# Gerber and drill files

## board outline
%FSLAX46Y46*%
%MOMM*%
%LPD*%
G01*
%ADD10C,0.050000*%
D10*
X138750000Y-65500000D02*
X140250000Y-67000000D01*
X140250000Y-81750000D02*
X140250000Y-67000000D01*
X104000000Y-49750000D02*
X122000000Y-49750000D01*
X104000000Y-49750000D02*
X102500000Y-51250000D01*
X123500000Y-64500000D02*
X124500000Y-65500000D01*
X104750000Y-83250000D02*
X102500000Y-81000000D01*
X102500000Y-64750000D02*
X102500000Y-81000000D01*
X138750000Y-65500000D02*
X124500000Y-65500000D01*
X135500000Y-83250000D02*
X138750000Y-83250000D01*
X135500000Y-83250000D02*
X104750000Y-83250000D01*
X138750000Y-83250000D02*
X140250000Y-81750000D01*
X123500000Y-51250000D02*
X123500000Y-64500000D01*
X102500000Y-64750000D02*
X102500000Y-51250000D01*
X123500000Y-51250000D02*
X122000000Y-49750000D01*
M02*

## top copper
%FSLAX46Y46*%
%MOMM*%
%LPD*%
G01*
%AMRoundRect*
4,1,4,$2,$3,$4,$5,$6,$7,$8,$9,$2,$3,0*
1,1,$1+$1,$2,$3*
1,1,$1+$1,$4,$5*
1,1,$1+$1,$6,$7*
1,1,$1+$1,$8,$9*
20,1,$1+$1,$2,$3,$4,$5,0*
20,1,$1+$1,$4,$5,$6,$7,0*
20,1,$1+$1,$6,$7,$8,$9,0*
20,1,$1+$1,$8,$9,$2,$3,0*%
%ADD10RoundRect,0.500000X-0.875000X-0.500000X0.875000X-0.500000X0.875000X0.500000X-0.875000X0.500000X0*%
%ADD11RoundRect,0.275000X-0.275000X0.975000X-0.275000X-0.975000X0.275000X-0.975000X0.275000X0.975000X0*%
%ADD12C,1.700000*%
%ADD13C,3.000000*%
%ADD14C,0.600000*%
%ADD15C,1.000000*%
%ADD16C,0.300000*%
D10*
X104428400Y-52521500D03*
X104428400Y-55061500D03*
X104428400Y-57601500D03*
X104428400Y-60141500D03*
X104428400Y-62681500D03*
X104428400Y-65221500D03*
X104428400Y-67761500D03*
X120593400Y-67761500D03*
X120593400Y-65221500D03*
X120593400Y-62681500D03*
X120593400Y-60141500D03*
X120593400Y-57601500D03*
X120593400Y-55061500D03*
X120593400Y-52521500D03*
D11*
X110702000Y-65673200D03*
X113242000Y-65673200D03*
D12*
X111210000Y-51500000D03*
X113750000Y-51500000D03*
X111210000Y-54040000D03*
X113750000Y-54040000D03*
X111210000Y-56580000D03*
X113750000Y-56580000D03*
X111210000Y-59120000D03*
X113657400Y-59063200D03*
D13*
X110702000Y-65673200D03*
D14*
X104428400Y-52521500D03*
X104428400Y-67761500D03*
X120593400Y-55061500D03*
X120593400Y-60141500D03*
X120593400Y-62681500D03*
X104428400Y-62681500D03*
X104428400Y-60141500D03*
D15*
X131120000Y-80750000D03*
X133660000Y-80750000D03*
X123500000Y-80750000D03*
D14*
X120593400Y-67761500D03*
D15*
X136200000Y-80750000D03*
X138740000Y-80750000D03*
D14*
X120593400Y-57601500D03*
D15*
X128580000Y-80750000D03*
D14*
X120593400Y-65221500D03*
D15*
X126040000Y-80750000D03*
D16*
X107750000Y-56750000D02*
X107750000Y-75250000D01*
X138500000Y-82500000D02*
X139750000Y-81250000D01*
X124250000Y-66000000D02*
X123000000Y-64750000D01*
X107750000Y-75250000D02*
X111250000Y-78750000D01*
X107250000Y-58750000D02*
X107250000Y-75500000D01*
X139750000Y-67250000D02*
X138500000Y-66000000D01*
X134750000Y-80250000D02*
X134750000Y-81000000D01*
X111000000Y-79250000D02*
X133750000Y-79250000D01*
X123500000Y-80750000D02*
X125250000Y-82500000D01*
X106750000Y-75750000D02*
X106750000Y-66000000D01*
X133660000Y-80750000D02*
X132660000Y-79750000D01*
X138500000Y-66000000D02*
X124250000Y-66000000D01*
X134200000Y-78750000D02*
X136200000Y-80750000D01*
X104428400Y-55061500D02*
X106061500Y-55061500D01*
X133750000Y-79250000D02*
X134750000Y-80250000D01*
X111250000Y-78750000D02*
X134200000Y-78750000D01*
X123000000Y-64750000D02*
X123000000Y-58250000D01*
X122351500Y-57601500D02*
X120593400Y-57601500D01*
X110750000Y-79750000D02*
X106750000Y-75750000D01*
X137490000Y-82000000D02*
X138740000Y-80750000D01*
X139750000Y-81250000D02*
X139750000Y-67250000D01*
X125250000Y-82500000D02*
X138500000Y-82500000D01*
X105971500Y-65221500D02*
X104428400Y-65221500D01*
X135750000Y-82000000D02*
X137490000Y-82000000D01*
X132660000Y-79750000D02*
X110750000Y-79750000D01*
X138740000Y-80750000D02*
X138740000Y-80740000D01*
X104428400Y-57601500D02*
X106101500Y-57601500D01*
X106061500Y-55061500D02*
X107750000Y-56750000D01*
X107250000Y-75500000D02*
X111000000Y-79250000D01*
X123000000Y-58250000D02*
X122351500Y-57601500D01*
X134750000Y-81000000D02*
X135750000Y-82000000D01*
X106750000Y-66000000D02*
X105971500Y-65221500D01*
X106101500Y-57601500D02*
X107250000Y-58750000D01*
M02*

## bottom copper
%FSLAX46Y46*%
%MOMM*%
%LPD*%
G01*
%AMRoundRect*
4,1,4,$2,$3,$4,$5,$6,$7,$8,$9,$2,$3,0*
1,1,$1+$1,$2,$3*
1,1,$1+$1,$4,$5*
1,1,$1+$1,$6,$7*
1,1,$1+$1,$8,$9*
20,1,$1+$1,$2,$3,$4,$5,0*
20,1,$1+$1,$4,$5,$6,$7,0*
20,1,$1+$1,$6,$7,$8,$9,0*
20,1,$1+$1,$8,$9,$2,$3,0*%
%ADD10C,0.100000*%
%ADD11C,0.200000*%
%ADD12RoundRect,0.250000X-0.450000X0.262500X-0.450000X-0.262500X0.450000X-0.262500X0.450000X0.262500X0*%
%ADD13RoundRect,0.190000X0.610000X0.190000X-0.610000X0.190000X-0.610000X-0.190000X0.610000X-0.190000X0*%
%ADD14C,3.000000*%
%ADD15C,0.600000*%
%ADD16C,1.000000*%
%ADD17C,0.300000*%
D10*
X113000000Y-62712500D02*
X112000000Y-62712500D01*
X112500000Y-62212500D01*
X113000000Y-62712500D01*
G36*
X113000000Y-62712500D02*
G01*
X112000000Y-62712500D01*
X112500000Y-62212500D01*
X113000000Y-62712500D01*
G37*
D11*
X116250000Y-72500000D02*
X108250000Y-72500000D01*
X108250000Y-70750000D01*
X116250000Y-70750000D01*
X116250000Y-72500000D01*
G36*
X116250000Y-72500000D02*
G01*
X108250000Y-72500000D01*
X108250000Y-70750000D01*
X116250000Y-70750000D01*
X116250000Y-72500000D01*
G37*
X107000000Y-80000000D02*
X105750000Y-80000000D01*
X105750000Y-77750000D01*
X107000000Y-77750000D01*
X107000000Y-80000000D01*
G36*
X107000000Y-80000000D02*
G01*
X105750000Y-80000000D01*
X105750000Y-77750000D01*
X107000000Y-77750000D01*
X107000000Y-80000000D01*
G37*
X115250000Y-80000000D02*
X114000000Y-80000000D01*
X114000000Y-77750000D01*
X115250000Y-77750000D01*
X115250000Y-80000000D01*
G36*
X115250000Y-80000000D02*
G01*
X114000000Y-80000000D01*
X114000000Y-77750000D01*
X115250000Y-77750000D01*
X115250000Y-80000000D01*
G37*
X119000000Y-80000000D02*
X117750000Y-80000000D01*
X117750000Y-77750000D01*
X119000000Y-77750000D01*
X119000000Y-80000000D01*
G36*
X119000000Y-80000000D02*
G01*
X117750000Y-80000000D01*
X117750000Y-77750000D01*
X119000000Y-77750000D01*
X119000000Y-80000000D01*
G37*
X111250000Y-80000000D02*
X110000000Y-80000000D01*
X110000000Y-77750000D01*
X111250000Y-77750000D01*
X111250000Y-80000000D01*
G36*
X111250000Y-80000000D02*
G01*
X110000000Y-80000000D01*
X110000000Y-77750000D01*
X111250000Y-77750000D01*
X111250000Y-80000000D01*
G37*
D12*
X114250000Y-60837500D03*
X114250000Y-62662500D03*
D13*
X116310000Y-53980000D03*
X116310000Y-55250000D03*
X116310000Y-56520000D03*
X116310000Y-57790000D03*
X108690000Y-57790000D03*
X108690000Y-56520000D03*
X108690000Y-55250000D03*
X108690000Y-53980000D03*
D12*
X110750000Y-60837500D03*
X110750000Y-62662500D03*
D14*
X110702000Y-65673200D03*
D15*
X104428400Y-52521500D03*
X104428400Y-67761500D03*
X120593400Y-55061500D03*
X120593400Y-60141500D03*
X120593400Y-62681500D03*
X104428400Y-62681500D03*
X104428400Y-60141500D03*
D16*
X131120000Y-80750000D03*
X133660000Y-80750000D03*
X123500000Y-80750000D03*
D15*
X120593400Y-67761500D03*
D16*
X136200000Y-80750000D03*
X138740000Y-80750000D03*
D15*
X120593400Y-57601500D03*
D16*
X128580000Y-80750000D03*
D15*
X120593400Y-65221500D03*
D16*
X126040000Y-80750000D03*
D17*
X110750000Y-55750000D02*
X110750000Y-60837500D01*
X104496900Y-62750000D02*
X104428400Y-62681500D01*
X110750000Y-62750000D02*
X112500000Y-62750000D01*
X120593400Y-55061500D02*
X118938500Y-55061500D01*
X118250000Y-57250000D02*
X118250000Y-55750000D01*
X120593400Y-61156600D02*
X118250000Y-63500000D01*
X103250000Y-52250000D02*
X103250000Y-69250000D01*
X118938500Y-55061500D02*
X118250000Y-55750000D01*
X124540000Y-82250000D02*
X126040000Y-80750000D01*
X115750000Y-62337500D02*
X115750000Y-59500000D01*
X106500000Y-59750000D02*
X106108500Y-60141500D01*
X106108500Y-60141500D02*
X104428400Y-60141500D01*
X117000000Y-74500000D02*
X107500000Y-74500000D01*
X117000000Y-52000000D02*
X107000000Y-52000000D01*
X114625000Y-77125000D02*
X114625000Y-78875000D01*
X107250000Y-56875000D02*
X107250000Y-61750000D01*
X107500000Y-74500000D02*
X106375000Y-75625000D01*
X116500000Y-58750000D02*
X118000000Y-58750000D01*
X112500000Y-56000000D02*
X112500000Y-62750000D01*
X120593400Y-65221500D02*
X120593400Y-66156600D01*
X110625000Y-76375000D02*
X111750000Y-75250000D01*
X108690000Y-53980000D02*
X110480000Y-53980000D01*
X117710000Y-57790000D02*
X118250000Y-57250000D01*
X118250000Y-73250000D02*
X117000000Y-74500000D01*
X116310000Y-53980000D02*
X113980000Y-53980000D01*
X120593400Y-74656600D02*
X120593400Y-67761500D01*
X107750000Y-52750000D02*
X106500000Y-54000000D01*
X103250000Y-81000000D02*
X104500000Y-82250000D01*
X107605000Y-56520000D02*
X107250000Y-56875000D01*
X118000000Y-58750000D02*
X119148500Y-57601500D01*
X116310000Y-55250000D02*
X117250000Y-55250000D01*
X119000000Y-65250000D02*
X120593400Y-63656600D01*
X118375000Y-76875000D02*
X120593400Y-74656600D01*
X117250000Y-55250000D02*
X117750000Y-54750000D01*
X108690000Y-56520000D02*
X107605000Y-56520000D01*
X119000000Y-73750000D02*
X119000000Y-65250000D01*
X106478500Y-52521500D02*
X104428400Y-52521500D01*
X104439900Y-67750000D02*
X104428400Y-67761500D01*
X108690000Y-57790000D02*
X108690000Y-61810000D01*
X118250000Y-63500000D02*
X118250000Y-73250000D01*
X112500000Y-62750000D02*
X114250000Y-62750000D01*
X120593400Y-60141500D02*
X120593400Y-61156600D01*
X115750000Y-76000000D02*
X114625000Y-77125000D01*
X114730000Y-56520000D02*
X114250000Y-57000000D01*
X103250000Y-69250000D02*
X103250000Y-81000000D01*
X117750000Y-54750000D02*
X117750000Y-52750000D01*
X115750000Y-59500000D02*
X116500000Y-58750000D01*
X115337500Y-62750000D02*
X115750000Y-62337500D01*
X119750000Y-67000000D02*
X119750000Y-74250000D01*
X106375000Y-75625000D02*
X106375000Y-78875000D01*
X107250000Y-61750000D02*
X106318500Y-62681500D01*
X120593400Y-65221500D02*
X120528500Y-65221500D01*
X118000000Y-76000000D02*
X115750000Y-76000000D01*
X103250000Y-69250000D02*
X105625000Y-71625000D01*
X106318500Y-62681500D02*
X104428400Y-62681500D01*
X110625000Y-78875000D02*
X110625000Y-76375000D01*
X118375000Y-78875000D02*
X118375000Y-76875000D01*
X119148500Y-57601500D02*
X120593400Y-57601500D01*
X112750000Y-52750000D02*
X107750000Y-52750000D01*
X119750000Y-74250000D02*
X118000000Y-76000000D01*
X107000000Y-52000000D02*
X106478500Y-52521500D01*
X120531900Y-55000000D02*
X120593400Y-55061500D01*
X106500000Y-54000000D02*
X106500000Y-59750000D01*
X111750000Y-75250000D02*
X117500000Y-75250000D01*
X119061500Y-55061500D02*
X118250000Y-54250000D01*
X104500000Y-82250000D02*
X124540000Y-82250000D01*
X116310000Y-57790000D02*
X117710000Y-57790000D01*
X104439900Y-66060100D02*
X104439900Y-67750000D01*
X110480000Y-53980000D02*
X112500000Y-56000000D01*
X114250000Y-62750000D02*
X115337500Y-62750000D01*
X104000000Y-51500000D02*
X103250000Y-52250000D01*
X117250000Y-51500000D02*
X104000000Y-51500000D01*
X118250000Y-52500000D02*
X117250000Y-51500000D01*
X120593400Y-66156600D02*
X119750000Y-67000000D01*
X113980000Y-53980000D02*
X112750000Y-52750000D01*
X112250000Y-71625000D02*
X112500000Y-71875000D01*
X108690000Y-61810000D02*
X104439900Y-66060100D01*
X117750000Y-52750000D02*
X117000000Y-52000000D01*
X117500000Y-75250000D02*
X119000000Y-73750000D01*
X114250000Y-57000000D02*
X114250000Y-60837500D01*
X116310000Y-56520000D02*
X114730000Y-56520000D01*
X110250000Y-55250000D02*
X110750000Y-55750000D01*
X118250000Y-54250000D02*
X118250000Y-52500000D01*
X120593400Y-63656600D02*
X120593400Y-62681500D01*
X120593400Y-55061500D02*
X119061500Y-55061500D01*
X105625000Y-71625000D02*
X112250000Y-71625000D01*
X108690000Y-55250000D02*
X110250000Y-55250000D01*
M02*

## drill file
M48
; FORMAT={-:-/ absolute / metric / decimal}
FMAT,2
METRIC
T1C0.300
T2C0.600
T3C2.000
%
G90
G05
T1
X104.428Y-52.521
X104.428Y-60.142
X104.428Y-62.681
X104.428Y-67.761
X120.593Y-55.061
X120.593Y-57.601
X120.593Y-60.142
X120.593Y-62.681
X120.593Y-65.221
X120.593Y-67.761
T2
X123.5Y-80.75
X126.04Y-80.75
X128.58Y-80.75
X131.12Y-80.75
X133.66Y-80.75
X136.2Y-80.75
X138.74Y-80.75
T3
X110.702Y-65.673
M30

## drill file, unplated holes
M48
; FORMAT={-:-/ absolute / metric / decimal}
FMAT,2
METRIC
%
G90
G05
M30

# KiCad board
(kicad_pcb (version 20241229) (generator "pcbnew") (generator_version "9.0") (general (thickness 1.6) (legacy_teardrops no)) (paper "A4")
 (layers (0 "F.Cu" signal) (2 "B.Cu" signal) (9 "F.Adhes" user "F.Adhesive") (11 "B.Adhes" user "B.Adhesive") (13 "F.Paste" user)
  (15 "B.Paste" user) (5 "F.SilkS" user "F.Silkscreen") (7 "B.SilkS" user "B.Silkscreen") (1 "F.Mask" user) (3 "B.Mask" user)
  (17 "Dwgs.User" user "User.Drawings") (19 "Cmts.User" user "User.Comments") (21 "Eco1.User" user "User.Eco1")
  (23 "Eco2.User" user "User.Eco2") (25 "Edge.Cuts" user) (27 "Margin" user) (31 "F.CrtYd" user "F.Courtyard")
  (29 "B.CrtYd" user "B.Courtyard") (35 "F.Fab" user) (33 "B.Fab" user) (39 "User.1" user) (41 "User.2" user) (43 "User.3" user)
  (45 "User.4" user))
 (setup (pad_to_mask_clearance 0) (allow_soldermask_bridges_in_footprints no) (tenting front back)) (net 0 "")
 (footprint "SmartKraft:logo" (layer "F.Cu") (at 131.25 71.25)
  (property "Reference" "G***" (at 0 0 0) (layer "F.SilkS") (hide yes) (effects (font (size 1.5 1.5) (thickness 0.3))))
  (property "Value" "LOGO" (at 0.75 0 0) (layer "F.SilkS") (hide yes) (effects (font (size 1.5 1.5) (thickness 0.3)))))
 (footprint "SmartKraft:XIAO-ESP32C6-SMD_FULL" (layer "F.Cu") (at 112.71 60.12)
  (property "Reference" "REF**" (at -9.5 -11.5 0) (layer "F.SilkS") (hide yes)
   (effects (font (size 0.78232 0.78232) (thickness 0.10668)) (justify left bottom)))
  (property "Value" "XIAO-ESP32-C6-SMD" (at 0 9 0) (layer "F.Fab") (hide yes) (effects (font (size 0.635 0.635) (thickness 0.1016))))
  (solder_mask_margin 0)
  (pad "1" smd roundrect (at -8.2816 -7.5985) (size 2.75 2) (layers "F.Cu" "F.Mask") (roundrect_rratio 0.25) (solder_mask_margin 0.0508)
   (thermal_bridge_angle 45))
  (pad "2" smd roundrect (at -8.2816 -5.0585) (size 2.75 2) (layers "F.Cu" "F.Mask") (roundrect_rratio 0.25) (solder_mask_margin 0.0508)
   (thermal_bridge_angle 45))
  (pad "3" smd roundrect (at -8.2816 -2.5185) (size 2.75 2) (layers "F.Cu" "F.Mask") (roundrect_rratio 0.25) (solder_mask_margin 0.0508)
   (thermal_bridge_angle 45))
  (pad "4" smd roundrect (at -8.2816 0.0215) (size 2.75 2) (layers "F.Cu" "F.Mask") (roundrect_rratio 0.25) (solder_mask_margin 0.0508)
   (thermal_bridge_angle 45))
  (pad "5" smd roundrect (at -8.2816 2.5615) (size 2.75 2) (layers "F.Cu" "F.Mask") (roundrect_rratio 0.25) (solder_mask_margin 0.0508)
   (thermal_bridge_angle 45))
  (pad "6" smd roundrect (at -8.2816 5.1015) (size 2.75 2) (layers "F.Cu" "F.Mask") (roundrect_rratio 0.25) (solder_mask_margin 0.0508)
   (thermal_bridge_angle 45))
  (pad "7" smd roundrect (at -8.2816 7.6415) (size 2.75 2) (layers "F.Cu" "F.Mask") (roundrect_rratio 0.25) (solder_mask_margin 0.0508)
   (thermal_bridge_angle 45))
  (pad "8" smd roundrect (at 7.8834 7.6415) (size 2.75 2) (layers "F.Cu" "F.Mask") (roundrect_rratio 0.25) (solder_mask_margin 0.0508)
   (thermal_bridge_angle 45))
  (pad "9" smd roundrect (at 7.8834 5.1015) (size 2.75 2) (layers "F.Cu" "F.Mask") (roundrect_rratio 0.25) (solder_mask_margin 0.0508)
   (thermal_bridge_angle 45))
  (pad "10" smd roundrect (at 7.8834 2.5615) (size 2.75 2) (layers "F.Cu" "F.Mask") (roundrect_rratio 0.25) (solder_mask_margin 0.0508)
   (thermal_bridge_angle 45))
  (pad "11" smd roundrect (at 7.8834 0.0215) (size 2.75 2) (layers "F.Cu" "F.Mask") (roundrect_rratio 0.25) (solder_mask_margin 0.0508)
   (thermal_bridge_angle 45))
  (pad "12" smd roundrect (at 7.8834 -2.5185) (size 2.75 2) (layers "F.Cu" "F.Mask") (roundrect_rratio 0.25) (solder_mask_margin 0.0508)
   (thermal_bridge_angle 45))
  (pad "13" smd roundrect (at 7.8834 -5.0585) (size 2.75 2) (layers "F.Cu" "F.Mask") (roundrect_rratio 0.25) (solder_mask_margin 0.0508)
   (thermal_bridge_angle 45))
  (pad "14" smd roundrect (at 7.8834 -7.5985) (size 2.75 2) (layers "F.Cu" "F.Mask") (roundrect_rratio 0.25) (solder_mask_margin 0.0508)
   (thermal_bridge_angle 45))
  (pad "15" smd roundrect (at -2.008 5.5532 270) (size 2.5 1.1) (layers "F.Cu" "F.Mask" "F.Paste") (roundrect_rratio 0.25)
   (solder_mask_margin 0.0508) (thermal_bridge_angle 45))
  (pad "16" smd roundrect (at 0.532 5.5532 270) (size 2.5 1.1) (layers "F.Cu" "F.Mask" "F.Paste") (roundrect_rratio 0.25)
   (solder_mask_margin 0.0508) (thermal_bridge_angle 45))
  (pad "17" smd circle (at -1.5 -8.62) (size 1.7 1.7) (layers "F.Cu" "F.Mask" "F.Paste"))
  (pad "18" smd circle (at 1.04 -8.62) (size 1.7 1.7) (layers "F.Cu" "F.Mask" "F.Paste"))
  (pad "19" smd circle (at -1.5 -6.08) (size 1.7 1.7) (layers "F.Cu" "F.Mask" "F.Paste"))
  (pad "20" smd circle (at 1.04 -6.08) (size 1.7 1.7) (layers "F.Cu" "F.Mask" "F.Paste"))
  (pad "21" smd circle (at -1.5 -3.54) (size 1.7 1.7) (layers "F.Cu" "F.Mask" "F.Paste"))
  (pad "22" smd circle (at 1.04 -3.54) (size 1.7 1.7) (layers "F.Cu" "F.Mask" "F.Paste"))
  (pad "23" smd circle (at -1.5 -1) (size 1.7 1.7) (layers "F.Cu" "F.Mask" "F.Paste"))
  (pad "24" smd circle (at 0.9474 -1.0568) (size 1.7 1.7) (layers "F.Cu" "F.Mask" "F.Paste")))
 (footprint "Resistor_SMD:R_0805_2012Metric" (layer "B.Cu") (at 114.25 61.75 -90)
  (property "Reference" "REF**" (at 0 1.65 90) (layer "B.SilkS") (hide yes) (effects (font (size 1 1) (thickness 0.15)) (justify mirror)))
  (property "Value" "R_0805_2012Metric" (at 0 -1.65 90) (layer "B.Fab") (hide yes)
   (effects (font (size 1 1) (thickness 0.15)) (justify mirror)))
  (pad "1" smd roundrect (at -0.9125 0 270) (size 1.025 1.4) (layers "B.Cu" "B.Mask") (roundrect_rratio 0.243902)
   (padstack (mode custom)
    (layer "B.Cu" (shape roundrect) (size 1.025 1.4) (roundrect_rratio 0.243902) (thermal_bridge_angle 45) (zone_connect -1))))
  (pad "2" smd roundrect (at 0.9125 0 270) (size 1.025 1.4) (layers "B.Cu" "B.Mask") (roundrect_rratio 0.243902)
   (padstack (mode custom)
    (layer "B.Cu" (shape roundrect) (size 1.025 1.4) (roundrect_rratio 0.243902) (thermal_bridge_angle 45) (zone_connect -1)))))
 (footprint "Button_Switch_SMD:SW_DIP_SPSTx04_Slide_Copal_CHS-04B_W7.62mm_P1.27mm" (layer "B.Cu") (at 112.5 55.885 180)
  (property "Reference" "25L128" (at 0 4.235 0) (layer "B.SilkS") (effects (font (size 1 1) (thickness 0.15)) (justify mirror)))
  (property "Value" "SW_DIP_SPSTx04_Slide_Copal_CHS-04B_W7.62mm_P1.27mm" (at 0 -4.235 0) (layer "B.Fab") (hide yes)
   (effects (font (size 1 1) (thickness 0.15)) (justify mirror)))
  (pad "1" smd roundrect (at -3.81 1.905 180) (size 1.6 0.76) (layers "B.Cu" "B.Mask") (roundrect_rratio 0.25))
  (pad "2" smd roundrect (at -3.81 0.635 180) (size 1.6 0.76) (layers "B.Cu" "B.Mask") (roundrect_rratio 0.25))
  (pad "3" smd roundrect (at -3.81 -0.635 180) (size 1.6 0.76) (layers "B.Cu" "B.Mask") (roundrect_rratio 0.25))
  (pad "4" smd roundrect (at -3.81 -1.905 180) (size 1.6 0.76) (layers "B.Cu" "B.Mask") (roundrect_rratio 0.25))
  (pad "5" smd roundrect (at 3.81 -1.905 180) (size 1.6 0.76) (layers "B.Cu" "B.Mask") (roundrect_rratio 0.25))
  (pad "6" smd roundrect (at 3.81 -0.635 180) (size 1.6 0.76) (layers "B.Cu" "B.Mask") (roundrect_rratio 0.25))
  (pad "7" smd roundrect (at 3.81 0.635 180) (size 1.6 0.76) (layers "B.Cu" "B.Mask") (roundrect_rratio 0.25))
  (pad "8" smd roundrect (at 3.81 1.905 180) (size 1.6 0.76) (layers "B.Cu" "B.Mask") (roundrect_rratio 0.25)))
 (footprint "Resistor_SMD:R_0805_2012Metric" (layer "B.Cu") (at 110.75 61.75 -90)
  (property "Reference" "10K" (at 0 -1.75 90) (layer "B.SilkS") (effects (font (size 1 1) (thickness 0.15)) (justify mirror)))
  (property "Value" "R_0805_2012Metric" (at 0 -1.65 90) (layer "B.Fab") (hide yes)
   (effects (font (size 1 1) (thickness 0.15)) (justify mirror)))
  (pad "1" smd roundrect (at -0.9125 0 270) (size 1.025 1.4) (layers "B.Cu" "B.Mask") (roundrect_rratio 0.243902)
   (padstack (mode custom)
    (layer "B.Cu" (shape roundrect) (size 1.025 1.4) (roundrect_rratio 0.243902) (thermal_bridge_angle 45) (zone_connect -1))))
  (pad "2" smd roundrect (at 0.9125 0 270) (size 1.025 1.4) (layers "B.Cu" "B.Mask") (roundrect_rratio 0.243902)
   (padstack (mode custom)
    (layer "B.Cu" (shape roundrect) (size 1.025 1.4) (roundrect_rratio 0.243902) (thermal_bridge_angle 45) (zone_connect -1)))))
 (gr_poly (pts (xy 112.5 62.2125) (xy 113 62.7125) (xy 112 62.7125)) (stroke (width 0.1) (type solid)) (fill yes) (layer "B.Cu"))
 (gr_poly
  (pts (xy 108.25 70.75) (xy 116.25 70.75) (xy 116.25 72.5) (xy 108.25 72.5)) (stroke (width 0.2) (type solid)) (fill yes)
  (layers "B.Cu" "B.Mask"))
 (gr_poly
  (pts (xy 107 77.75) (xy 107 80) (xy 105.75 80) (xy 105.75 77.75)) (stroke (width 0.2) (type solid)) (fill yes) (layers "B.Cu" "B.Mask"))
 (gr_poly
  (pts (xy 115.25 77.75) (xy 115.25 80) (xy 114 80) (xy 114 77.75)) (stroke (width 0.2) (type solid)) (fill yes) (layers "B.Cu" "B.Mask"))
 (gr_poly
  (pts (xy 119 77.75) (xy 119 80) (xy 117.75 80) (xy 117.75 77.75)) (stroke (width 0.2) (type solid)) (fill yes) (layers "B.Cu" "B.Mask"))
 (gr_poly
  (pts (xy 111.25 77.75) (xy 111.25 80) (xy 110 80) (xy 110 77.75)) (stroke (width 0.2) (type solid)) (fill yes) (layers "B.Cu" "B.Mask"))
 (gr_line (start 138.75 65.5) (end 140.25 67) (stroke (width 0.05) (type default)) (layer "Edge.Cuts"))
 (gr_line (start 140.25 81.75) (end 140.25 67) (stroke (width 0.05) (type default)) (layer "Edge.Cuts"))
 (gr_line (start 104 49.75) (end 122 49.75) (stroke (width 0.05) (type default)) (layer "Edge.Cuts"))
 (gr_line (start 104 49.75) (end 102.5 51.25) (stroke (width 0.05) (type default)) (layer "Edge.Cuts"))
 (gr_line (start 123.5 64.5) (end 124.5 65.5) (stroke (width 0.05) (type default)) (layer "Edge.Cuts"))
 (gr_line (start 104.75 83.25) (end 102.5 81) (stroke (width 0.05) (type default)) (layer "Edge.Cuts"))
 (gr_line (start 102.5 64.75) (end 102.5 81) (stroke (width 0.05) (type default)) (layer "Edge.Cuts"))
 (gr_line (start 138.75 65.5) (end 124.5 65.5) (stroke (width 0.05) (type default)) (layer "Edge.Cuts"))
 (gr_line (start 135.5 83.25) (end 138.75 83.25) (stroke (width 0.05) (type default)) (layer "Edge.Cuts"))
 (gr_line (start 135.5 83.25) (end 104.75 83.25) (stroke (width 0.05) (type default)) (layer "Edge.Cuts"))
 (gr_line (start 138.75 83.25) (end 140.25 81.75) (stroke (width 0.05) (type default)) (layer "Edge.Cuts"))
 (gr_line (start 123.5 51.25) (end 123.5 64.5) (stroke (width 0.05) (type default)) (layer "Edge.Cuts"))
 (gr_line (start 102.5 64.75) (end 102.5 51.25) (stroke (width 0.05) (type default)) (layer "Edge.Cuts"))
 (gr_line (start 123.5 51.25) (end 122 49.75) (stroke (width 0.05) (type default)) (layer "Edge.Cuts"))
 (segment (start 107.75 56.75) (end 107.75 75.25) (width 0.3) (layer "F.Cu") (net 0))
 (segment (start 138.5 82.5) (end 139.75 81.25) (width 0.3) (layer "F.Cu") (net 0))
 (segment (start 124.25 66) (end 123 64.75) (width 0.3) (layer "F.Cu") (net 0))
 (segment (start 107.75 75.25) (end 111.25 78.75) (width 0.3) (layer "F.Cu") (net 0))
 (segment (start 107.25 58.75) (end 107.25 75.5) (width 0.3) (layer "F.Cu") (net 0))
 (segment (start 139.75 67.25) (end 138.5 66) (width 0.3) (layer "F.Cu") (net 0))
 (segment (start 134.75 80.25) (end 134.75 81) (width 0.3) (layer "F.Cu") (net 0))
 (segment (start 111 79.25) (end 133.75 79.25) (width 0.3) (layer "F.Cu") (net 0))
 (segment (start 123.5 80.75) (end 125.25 82.5) (width 0.3) (layer "F.Cu") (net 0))
 (segment (start 106.75 75.75) (end 106.75 66) (width 0.3) (layer "F.Cu") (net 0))
 (segment (start 133.66 80.75) (end 132.66 79.75) (width 0.3) (layer "F.Cu") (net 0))
 (segment (start 138.5 66) (end 124.25 66) (width 0.3) (layer "F.Cu") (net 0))
 (segment (start 134.2 78.75) (end 136.2 80.75) (width 0.3) (layer "F.Cu") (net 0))
 (segment (start 104.4284 55.0615) (end 106.0615 55.0615) (width 0.3) (layer "F.Cu") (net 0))
 (segment (start 133.75 79.25) (end 134.75 80.25) (width 0.3) (layer "F.Cu") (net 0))
 (segment (start 111.25 78.75) (end 134.2 78.75) (width 0.3) (layer "F.Cu") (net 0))
 (segment (start 123 64.75) (end 123 58.25) (width 0.3) (layer "F.Cu") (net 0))
 (segment (start 122.3515 57.6015) (end 120.5934 57.6015) (width 0.3) (layer "F.Cu") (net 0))
 (segment (start 110.75 79.75) (end 106.75 75.75) (width 0.3) (layer "F.Cu") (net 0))
 (segment (start 137.49 82) (end 138.74 80.75) (width 0.3) (layer "F.Cu") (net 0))
 (segment (start 139.75 81.25) (end 139.75 67.25) (width 0.3) (layer "F.Cu") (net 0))
 (segment (start 125.25 82.5) (end 138.5 82.5) (width 0.3) (layer "F.Cu") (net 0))
 (segment (start 105.9715 65.2215) (end 104.4284 65.2215) (width 0.3) (layer "F.Cu") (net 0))
 (segment (start 135.75 82) (end 137.49 82) (width 0.3) (layer "F.Cu") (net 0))
 (segment (start 132.66 79.75) (end 110.75 79.75) (width 0.3) (layer "F.Cu") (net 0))
 (segment (start 138.74 80.75) (end 138.74 80.74) (width 0.3) (layer "F.Cu") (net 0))
 (segment (start 104.4284 57.6015) (end 106.1015 57.6015) (width 0.3) (layer "F.Cu") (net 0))
 (segment (start 106.0615 55.0615) (end 107.75 56.75) (width 0.3) (layer "F.Cu") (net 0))
 (segment (start 107.25 75.5) (end 111 79.25) (width 0.3) (layer "F.Cu") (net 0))
 (segment (start 123 58.25) (end 122.3515 57.6015) (width 0.3) (layer "F.Cu") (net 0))
 (segment (start 134.75 81) (end 135.75 82) (width 0.3) (layer "F.Cu") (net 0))
 (segment (start 106.75 66) (end 105.9715 65.2215) (width 0.3) (layer "F.Cu") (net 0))
 (segment (start 106.1015 57.6015) (end 107.25 58.75) (width 0.3) (layer "F.Cu") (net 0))
 (via (at 104.4284 52.5215) (size 0.6) (drill 0.3) (layers "F.Cu" "B.Cu") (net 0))
 (via (at 104.4284 67.7615) (size 0.6) (drill 0.3) (layers "F.Cu" "B.Cu") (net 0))
 (via (at 120.5934 55.0615) (size 0.6) (drill 0.3) (layers "F.Cu" "B.Cu") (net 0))
 (via (at 120.5934 60.1415) (size 0.6) (drill 0.3) (layers "F.Cu" "B.Cu") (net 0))
 (via (at 120.5934 62.6815) (size 0.6) (drill 0.3) (layers "F.Cu" "B.Cu") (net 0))
 (via (at 104.4284 62.6815) (size 0.6) (drill 0.3) (layers "F.Cu" "B.Cu") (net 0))
 (via (at 104.4284 60.1415) (size 0.6) (drill 0.3) (layers "F.Cu" "B.Cu") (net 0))
 (via (at 131.12 80.75) (size 1) (drill 0.6) (layers "F.Cu" "B.Cu") (tenting none) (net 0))
 (via (at 110.702 65.6732) (size 3) (drill 2) (layers "F.Cu" "B.Cu") (tenting none) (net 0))
 (via (at 133.66 80.75) (size 1) (drill 0.6) (layers "F.Cu" "B.Cu") (tenting none) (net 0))
 (via (at 123.5 80.75) (size 1) (drill 0.6) (layers "F.Cu" "B.Cu") (tenting none) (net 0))
 (via (at 120.5934 67.7615) (size 0.6) (drill 0.3) (layers "F.Cu" "B.Cu") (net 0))
 (via (at 136.2 80.75) (size 1) (drill 0.6) (layers "F.Cu" "B.Cu") (tenting none) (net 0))
 (via (at 138.74 80.75) (size 1) (drill 0.6) (layers "F.Cu" "B.Cu") (tenting none) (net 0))
 (via (at 120.5934 57.6015) (size 0.6) (drill 0.3) (layers "F.Cu" "B.Cu") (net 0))
 (via (at 128.58 80.75) (size 1) (drill 0.6) (layers "F.Cu" "B.Cu") (tenting none) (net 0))
 (via (at 120.5934 65.2215) (size 0.6) (drill 0.3) (layers "F.Cu" "B.Cu") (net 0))
 (via (at 126.04 80.75) (size 1) (drill 0.6) (layers "F.Cu" "B.Cu") (tenting none) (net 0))
 (segment (start 110.75 55.75) (end 110.75 60.8375) (width 0.3) (layer "B.Cu") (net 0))
 (segment (start 104.4969 62.75) (end 104.4284 62.6815) (width 0.3) (layer "B.Cu") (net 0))
 (segment (start 110.75 62.75) (end 112.5 62.75) (width 0.3) (layer "B.Cu") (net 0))
 (segment (start 120.5934 55.0615) (end 118.9385 55.0615) (width 0.3) (layer "B.Cu") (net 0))
 (segment (start 118.25 57.25) (end 118.25 55.75) (width 0.3) (layer "B.Cu") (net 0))
 (segment (start 120.5934 61.1566) (end 118.25 63.5) (width 0.3) (layer "B.Cu") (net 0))
 (segment (start 103.25 52.25) (end 103.25 69.25) (width 0.3) (layer "B.Cu") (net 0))
 (segment (start 118.9385 55.0615) (end 118.25 55.75) (width 0.3) (layer "B.Cu") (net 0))
 (segment (start 124.54 82.25) (end 126.04 80.75) (width 0.3) (layer "B.Cu") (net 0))
 (segment (start 115.75 62.3375) (end 115.75 59.5) (width 0.3) (layer "B.Cu") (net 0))
 (segment (start 106.5 59.75) (end 106.1085 60.1415) (width 0.3) (layer "B.Cu") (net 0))
 (segment (start 106.1085 60.1415) (end 104.4284 60.1415) (width 0.3) (layer "B.Cu") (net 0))
 (segment (start 117 74.5) (end 107.5 74.5) (width 0.3) (layer "B.Cu") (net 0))
 (segment (start 117 52) (end 107 52) (width 0.3) (layer "B.Cu") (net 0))
 (segment (start 114.625 77.125) (end 114.625 78.875) (width 0.3) (layer "B.Cu") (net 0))
 (segment (start 107.25 56.875) (end 107.25 61.75) (width 0.3) (layer "B.Cu") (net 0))
 (segment (start 107.5 74.5) (end 106.375 75.625) (width 0.3) (layer "B.Cu") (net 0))
 (segment (start 116.5 58.75) (end 118 58.75) (width 0.3) (layer "B.Cu") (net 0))
 (segment (start 112.5 56) (end 112.5 62.75) (width 0.3) (layer "B.Cu") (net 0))
 (segment (start 120.5934 65.2215) (end 120.5934 66.1566) (width 0.3) (layer "B.Cu") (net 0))
 (segment (start 110.625 76.375) (end 111.75 75.25) (width 0.3) (layer "B.Cu") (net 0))
 (segment (start 108.69 53.98) (end 110.48 53.98) (width 0.3) (layer "B.Cu") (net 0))
 (segment (start 117.71 57.79) (end 118.25 57.25) (width 0.3) (layer "B.Cu") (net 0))
 (segment (start 118.25 73.25) (end 117 74.5) (width 0.3) (layer "B.Cu") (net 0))
 (segment (start 116.31 53.98) (end 113.98 53.98) (width 0.3) (layer "B.Cu") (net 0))
 (segment (start 120.5934 74.6566) (end 120.5934 67.7615) (width 0.3) (layer "B.Cu") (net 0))
 (segment (start 107.75 52.75) (end 106.5 54) (width 0.3) (layer "B.Cu") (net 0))
 (segment (start 103.25 81) (end 104.5 82.25) (width 0.3) (layer "B.Cu") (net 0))
 (segment (start 107.605 56.52) (end 107.25 56.875) (width 0.3) (layer "B.Cu") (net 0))
 (segment (start 118 58.75) (end 119.1485 57.6015) (width 0.3) (layer "B.Cu") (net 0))
 (segment (start 116.31 55.25) (end 117.25 55.25) (width 0.3) (layer "B.Cu") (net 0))
 (segment (start 119 65.25) (end 120.5934 63.6566) (width 0.3) (layer "B.Cu") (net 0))
 (segment (start 118.375 76.875) (end 120.5934 74.6566) (width 0.3) (layer "B.Cu") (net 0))
 (segment (start 117.25 55.25) (end 117.75 54.75) (width 0.3) (layer "B.Cu") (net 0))
 (segment (start 108.69 56.52) (end 107.605 56.52) (width 0.3) (layer "B.Cu") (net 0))
 (segment (start 119 73.75) (end 119 65.25) (width 0.3) (layer "B.Cu") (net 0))
 (segment (start 106.4785 52.5215) (end 104.4284 52.5215) (width 0.3) (layer "B.Cu") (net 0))
 (segment (start 104.4399 67.75) (end 104.4284 67.7615) (width 0.3) (layer "B.Cu") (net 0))
 (segment (start 108.69 57.79) (end 108.69 61.81) (width 0.3) (layer "B.Cu") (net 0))
 (segment (start 118.25 63.5) (end 118.25 73.25) (width 0.3) (layer "B.Cu") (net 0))
 (segment (start 112.5 62.75) (end 114.25 62.75) (width 0.3) (layer "B.Cu") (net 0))
 (segment (start 120.5934 60.1415) (end 120.5934 61.1566) (width 0.3) (layer "B.Cu") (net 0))
 (segment (start 115.75 76) (end 114.625 77.125) (width 0.3) (layer "B.Cu") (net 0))
 (segment (start 114.73 56.52) (end 114.25 57) (width 0.3) (layer "B.Cu") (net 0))
 (segment (start 103.25 69.25) (end 103.25 81) (width 0.3) (layer "B.Cu") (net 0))
 (segment (start 117.75 54.75) (end 117.75 52.75) (width 0.3) (layer "B.Cu") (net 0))
 (segment (start 115.75 59.5) (end 116.5 58.75) (width 0.3) (layer "B.Cu") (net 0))
 (segment (start 115.3375 62.75) (end 115.75 62.3375) (width 0.3) (layer "B.Cu") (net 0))
 (segment (start 119.75 67) (end 119.75 74.25) (width 0.3) (layer "B.Cu") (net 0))
 (segment (start 106.375 75.625) (end 106.375 78.875) (width 0.3) (layer "B.Cu") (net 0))
 (segment (start 107.25 61.75) (end 106.3185 62.6815) (width 0.3) (layer "B.Cu") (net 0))
 (segment (start 120.5934 65.2215) (end 120.5285 65.2215) (width 0.3) (layer "B.Cu") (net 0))
 (segment (start 118 76) (end 115.75 76) (width 0.3) (layer "B.Cu") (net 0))
 (segment (start 103.25 69.25) (end 105.625 71.625) (width 0.3) (layer "B.Cu") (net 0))
 (segment (start 106.3185 62.6815) (end 104.4284 62.6815) (width 0.3) (layer "B.Cu") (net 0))
 (segment (start 110.625 78.875) (end 110.625 76.375) (width 0.3) (layer "B.Cu") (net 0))
 (segment (start 118.375 78.875) (end 118.375 76.875) (width 0.3) (layer "B.Cu") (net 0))
 (segment (start 119.1485 57.6015) (end 120.5934 57.6015) (width 0.3) (layer "B.Cu") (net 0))
 (segment (start 112.75 52.75) (end 107.75 52.75) (width 0.3) (layer "B.Cu") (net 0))
 (segment (start 119.75 74.25) (end 118 76) (width 0.3) (layer "B.Cu") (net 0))
 (segment (start 107 52) (end 106.4785 52.5215) (width 0.3) (layer "B.Cu") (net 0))
 (segment (start 120.5319 55) (end 120.5934 55.0615) (width 0.3) (layer "B.Cu") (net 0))
 (segment (start 106.5 54) (end 106.5 59.75) (width 0.3) (layer "B.Cu") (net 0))
 (segment (start 111.75 75.25) (end 117.5 75.25) (width 0.3) (layer "B.Cu") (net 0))
 (segment (start 119.0615 55.0615) (end 118.25 54.25) (width 0.3) (layer "B.Cu") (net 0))
 (segment (start 104.5 82.25) (end 124.54 82.25) (width 0.3) (layer "B.Cu") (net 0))
 (segment (start 116.31 57.79) (end 117.71 57.79) (width 0.3) (layer "B.Cu") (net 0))
 (segment (start 104.4399 66.0601) (end 104.4399 67.75) (width 0.3) (layer "B.Cu") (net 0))
 (segment (start 110.48 53.98) (end 112.5 56) (width 0.3) (layer "B.Cu") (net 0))
 (segment (start 114.25 62.75) (end 115.3375 62.75) (width 0.3) (layer "B.Cu") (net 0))
 (segment (start 104 51.5) (end 103.25 52.25) (width 0.3) (layer "B.Cu") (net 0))
 (segment (start 117.25 51.5) (end 104 51.5) (width 0.3) (layer "B.Cu") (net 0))
 (segment (start 118.25 52.5) (end 117.25 51.5) (width 0.3) (layer "B.Cu") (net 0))
 (segment (start 120.5934 66.1566) (end 119.75 67) (width 0.3) (layer "B.Cu") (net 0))
 (segment (start 113.98 53.98) (end 112.75 52.75) (width 0.3) (layer "B.Cu") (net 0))
 (segment (start 112.25 71.625) (end 112.5 71.875) (width 0.3) (layer "B.Cu") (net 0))
 (segment (start 108.69 61.81) (end 104.4399 66.0601) (width 0.3) (layer "B.Cu") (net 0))
 (segment (start 117.75 52.75) (end 117 52) (width 0.3) (layer "B.Cu") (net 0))
 (segment (start 117.5 75.25) (end 119 73.75) (width 0.3) (layer "B.Cu") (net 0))
 (segment (start 114.25 57) (end 114.25 60.8375) (width 0.3) (layer "B.Cu") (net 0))
 (segment (start 116.31 56.52) (end 114.73 56.52) (width 0.3) (layer "B.Cu") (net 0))
 (segment (start 110.25 55.25) (end 110.75 55.75) (width 0.3) (layer "B.Cu") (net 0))
 (segment (start 118.25 54.25) (end 118.25 52.5) (width 0.3) (layer "B.Cu") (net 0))
 (segment (start 120.5934 63.6566) (end 120.5934 62.6815) (width 0.3) (layer "B.Cu") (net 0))
 (segment (start 120.5934 55.0615) (end 119.0615 55.0615) (width 0.3) (layer "B.Cu") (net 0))
 (segment (start 105.625 71.625) (end 112.25 71.625) (width 0.3) (layer "B.Cu") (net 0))
 (segment (start 108.69 55.25) (end 110.25 55.25) (width 0.3) (layer "B.Cu") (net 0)))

